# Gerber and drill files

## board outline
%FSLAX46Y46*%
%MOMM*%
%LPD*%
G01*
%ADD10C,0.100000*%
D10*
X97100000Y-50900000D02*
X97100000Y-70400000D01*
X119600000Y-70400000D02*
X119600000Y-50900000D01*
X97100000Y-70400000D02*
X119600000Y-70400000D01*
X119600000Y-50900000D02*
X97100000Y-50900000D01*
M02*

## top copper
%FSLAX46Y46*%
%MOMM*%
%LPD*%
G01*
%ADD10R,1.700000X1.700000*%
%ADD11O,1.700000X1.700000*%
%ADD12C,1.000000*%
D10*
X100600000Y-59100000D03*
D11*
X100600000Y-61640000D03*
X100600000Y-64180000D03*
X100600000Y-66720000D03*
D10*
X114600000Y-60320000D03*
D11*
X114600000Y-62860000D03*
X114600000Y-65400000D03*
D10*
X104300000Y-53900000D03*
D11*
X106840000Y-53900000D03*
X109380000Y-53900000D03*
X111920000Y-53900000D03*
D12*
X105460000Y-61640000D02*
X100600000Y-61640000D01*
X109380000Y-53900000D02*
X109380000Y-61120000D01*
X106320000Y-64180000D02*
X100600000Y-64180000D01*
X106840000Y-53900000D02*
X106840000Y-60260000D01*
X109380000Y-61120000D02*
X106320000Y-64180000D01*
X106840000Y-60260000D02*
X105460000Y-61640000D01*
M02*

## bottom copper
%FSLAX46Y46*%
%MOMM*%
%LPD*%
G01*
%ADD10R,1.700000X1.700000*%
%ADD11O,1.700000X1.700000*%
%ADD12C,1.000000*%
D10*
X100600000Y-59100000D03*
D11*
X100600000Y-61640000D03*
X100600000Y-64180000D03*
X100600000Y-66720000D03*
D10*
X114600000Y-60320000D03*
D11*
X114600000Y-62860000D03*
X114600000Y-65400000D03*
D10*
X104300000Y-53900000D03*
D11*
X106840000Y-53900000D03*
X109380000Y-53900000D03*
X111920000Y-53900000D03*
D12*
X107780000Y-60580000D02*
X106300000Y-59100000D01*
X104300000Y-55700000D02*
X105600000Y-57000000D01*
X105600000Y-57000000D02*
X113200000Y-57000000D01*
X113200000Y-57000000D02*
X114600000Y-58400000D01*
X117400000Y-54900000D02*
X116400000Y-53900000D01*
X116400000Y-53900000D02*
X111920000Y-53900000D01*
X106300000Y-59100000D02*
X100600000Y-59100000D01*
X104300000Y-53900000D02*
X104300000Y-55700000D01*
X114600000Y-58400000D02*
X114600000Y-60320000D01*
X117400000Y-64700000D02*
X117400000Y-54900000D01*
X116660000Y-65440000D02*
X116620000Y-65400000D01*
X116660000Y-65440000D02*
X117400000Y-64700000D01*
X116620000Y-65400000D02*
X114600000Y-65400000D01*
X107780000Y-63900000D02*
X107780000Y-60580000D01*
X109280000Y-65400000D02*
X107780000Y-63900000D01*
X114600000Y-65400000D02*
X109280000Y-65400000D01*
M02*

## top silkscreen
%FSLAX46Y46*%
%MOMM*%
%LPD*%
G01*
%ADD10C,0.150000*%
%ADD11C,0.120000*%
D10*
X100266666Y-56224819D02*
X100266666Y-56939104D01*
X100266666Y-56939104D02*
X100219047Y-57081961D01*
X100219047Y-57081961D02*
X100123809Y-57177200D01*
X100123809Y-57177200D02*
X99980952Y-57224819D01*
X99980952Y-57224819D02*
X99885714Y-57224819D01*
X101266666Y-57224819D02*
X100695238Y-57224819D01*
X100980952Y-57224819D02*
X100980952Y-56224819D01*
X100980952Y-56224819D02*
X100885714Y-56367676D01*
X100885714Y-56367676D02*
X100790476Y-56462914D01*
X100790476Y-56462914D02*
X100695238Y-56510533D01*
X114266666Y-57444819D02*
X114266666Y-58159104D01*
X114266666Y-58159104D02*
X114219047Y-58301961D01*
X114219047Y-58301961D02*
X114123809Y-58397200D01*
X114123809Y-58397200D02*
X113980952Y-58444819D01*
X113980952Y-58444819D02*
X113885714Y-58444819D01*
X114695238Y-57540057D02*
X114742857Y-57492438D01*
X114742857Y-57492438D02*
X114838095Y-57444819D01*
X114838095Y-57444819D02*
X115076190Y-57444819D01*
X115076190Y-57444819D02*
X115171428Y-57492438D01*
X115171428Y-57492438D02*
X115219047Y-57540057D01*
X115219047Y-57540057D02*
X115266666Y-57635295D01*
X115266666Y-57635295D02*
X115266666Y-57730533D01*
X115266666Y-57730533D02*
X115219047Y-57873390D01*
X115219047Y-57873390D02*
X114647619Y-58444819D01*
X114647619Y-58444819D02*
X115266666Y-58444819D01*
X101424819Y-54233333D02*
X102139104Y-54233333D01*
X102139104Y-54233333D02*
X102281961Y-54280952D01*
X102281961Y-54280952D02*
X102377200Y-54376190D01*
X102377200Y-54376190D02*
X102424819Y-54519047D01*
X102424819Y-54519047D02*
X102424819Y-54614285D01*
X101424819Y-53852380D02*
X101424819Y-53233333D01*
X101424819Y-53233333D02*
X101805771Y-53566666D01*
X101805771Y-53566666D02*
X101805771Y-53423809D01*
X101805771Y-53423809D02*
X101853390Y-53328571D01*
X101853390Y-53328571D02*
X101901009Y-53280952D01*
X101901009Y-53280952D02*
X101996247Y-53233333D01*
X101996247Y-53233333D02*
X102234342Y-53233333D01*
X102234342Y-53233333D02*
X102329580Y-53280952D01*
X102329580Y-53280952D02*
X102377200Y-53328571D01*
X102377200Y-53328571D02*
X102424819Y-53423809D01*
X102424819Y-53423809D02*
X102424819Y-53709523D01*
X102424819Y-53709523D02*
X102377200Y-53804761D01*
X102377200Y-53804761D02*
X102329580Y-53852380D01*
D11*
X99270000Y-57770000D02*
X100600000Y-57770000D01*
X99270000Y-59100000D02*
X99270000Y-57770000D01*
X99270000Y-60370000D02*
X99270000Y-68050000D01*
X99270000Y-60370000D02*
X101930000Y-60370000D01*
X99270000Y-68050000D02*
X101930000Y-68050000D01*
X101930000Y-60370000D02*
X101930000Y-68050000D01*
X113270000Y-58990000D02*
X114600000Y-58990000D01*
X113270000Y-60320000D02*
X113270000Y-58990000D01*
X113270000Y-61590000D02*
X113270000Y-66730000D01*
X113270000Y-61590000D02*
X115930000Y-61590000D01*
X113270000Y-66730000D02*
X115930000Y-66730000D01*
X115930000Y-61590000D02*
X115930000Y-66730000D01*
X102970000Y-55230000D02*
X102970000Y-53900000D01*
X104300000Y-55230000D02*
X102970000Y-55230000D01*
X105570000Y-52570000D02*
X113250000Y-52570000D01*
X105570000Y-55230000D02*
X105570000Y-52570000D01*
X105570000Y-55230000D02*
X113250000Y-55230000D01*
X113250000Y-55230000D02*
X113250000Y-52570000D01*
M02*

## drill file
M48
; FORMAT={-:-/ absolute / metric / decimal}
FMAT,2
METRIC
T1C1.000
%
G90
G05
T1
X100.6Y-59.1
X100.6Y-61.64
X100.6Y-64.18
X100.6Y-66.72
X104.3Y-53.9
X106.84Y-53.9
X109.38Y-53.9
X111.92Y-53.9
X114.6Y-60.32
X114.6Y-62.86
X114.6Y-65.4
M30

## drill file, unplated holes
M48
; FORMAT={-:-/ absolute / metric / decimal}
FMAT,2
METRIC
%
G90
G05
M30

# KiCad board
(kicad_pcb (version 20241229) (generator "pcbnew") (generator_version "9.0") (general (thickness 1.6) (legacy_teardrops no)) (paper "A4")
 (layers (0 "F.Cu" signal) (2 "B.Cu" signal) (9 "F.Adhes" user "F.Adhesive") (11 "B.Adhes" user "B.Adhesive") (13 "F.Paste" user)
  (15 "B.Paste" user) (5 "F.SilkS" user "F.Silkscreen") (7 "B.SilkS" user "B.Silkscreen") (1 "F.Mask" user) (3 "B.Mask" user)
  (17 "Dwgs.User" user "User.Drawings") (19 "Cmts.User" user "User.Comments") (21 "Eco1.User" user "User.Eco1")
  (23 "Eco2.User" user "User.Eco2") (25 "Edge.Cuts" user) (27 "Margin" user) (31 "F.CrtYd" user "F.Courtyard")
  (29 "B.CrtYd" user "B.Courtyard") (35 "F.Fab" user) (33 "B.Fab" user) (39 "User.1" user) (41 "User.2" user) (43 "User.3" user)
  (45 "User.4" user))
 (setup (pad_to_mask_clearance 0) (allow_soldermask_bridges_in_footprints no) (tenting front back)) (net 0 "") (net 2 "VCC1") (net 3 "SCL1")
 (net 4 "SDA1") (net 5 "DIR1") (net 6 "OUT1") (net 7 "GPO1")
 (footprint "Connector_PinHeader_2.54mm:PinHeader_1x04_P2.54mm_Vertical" (layer "F.Cu") (at 104.3 53.9 90)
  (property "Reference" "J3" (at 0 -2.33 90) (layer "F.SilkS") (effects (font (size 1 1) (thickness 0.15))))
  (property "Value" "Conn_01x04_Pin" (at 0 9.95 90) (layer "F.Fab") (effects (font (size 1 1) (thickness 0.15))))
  (fp_line (start -1.33 -1.33) (end 0 -1.33) (stroke (width 0.12) (type solid)) (layer "F.SilkS") (net 1))
  (fp_line (start -1.33 0) (end -1.33 -1.33) (stroke (width 0.12) (type solid)) (layer "F.SilkS") (net 1))
  (fp_line (start 1.33 1.27) (end 1.33 8.95) (stroke (width 0.12) (type solid)) (layer "F.SilkS") (net 1))
  (fp_line (start -1.33 1.27) (end 1.33 1.27) (stroke (width 0.12) (type solid)) (layer "F.SilkS") (net 1))
  (fp_line (start -1.33 1.27) (end -1.33 8.95) (stroke (width 0.12) (type solid)) (layer "F.SilkS") (net 1))
  (fp_line (start -1.33 8.95) (end 1.33 8.95) (stroke (width 0.12) (type solid)) (layer "F.SilkS") (net 1))
  (pad "1" thru_hole rect (at 0 0 90) (size 1.7 1.7) (drill 1) (layers "*.Cu" "*.Mask") (remove_unused_layers no) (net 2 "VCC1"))
  (pad "2" thru_hole oval (at 0 2.54 90) (size 1.7 1.7) (drill 1) (layers "*.Cu" "*.Mask") (remove_unused_layers no) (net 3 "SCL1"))
  (pad "3" thru_hole oval (at 0 5.08 90) (size 1.7 1.7) (drill 1) (layers "*.Cu" "*.Mask") (remove_unused_layers no) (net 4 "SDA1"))
  (pad "4" thru_hole oval (at 0 7.62 90) (size 1.7 1.7) (drill 1) (layers "*.Cu" "*.Mask") (remove_unused_layers no) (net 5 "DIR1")))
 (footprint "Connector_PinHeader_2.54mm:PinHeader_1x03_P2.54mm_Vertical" (layer "F.Cu") (at 114.6 60.32)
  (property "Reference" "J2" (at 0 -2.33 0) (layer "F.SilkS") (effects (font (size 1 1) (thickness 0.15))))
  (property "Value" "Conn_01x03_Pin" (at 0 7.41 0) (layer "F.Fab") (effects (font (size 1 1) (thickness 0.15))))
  (fp_line (start -1.33 -1.33) (end 0 -1.33) (stroke (width 0.12) (type solid)) (layer "F.SilkS") (net 1))
  (fp_line (start -1.33 0) (end -1.33 -1.33) (stroke (width 0.12) (type solid)) (layer "F.SilkS") (net 1))
  (fp_line (start -1.33 1.27) (end -1.33 6.41) (stroke (width 0.12) (type solid)) (layer "F.SilkS") (net 1))
  (fp_line (start -1.33 1.27) (end 1.33 1.27) (stroke (width 0.12) (type solid)) (layer "F.SilkS") (net 1))
  (fp_line (start -1.33 6.41) (end 1.33 6.41) (stroke (width 0.12) (type solid)) (layer "F.SilkS") (net 1))
  (fp_line (start 1.33 1.27) (end 1.33 6.41) (stroke (width 0.12) (type solid)) (layer "F.SilkS") (net 1))
  (pad "1" thru_hole rect (at 0 0) (size 1.7 1.7) (drill 1) (layers "*.Cu" "*.Mask") (remove_unused_layers no) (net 2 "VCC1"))
  (pad "2" thru_hole oval (at 0 2.54) (size 1.7 1.7) (drill 1) (layers "*.Cu" "*.Mask") (remove_unused_layers no) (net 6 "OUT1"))
  (pad "3" thru_hole oval (at 0 5.08) (size 1.7 1.7) (drill 1) (layers "*.Cu" "*.Mask") (remove_unused_layers no) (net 5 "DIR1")))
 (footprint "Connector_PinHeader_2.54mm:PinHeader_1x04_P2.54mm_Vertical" (layer "F.Cu") (at 100.6 59.1)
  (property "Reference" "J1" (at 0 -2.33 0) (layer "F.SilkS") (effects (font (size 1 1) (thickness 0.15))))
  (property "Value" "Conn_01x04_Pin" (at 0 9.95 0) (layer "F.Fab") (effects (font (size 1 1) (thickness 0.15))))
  (fp_line (start -1.33 -1.33) (end 0 -1.33) (stroke (width 0.12) (type solid)) (layer "F.SilkS") (net 1))
  (fp_line (start -1.33 0) (end -1.33 -1.33) (stroke (width 0.12) (type solid)) (layer "F.SilkS") (net 1))
  (fp_line (start -1.33 1.27) (end -1.33 8.95) (stroke (width 0.12) (type solid)) (layer "F.SilkS") (net 1))
  (fp_line (start -1.33 1.27) (end 1.33 1.27) (stroke (width 0.12) (type solid)) (layer "F.SilkS") (net 1))
  (fp_line (start -1.33 8.95) (end 1.33 8.95) (stroke (width 0.12) (type solid)) (layer "F.SilkS") (net 1))
  (fp_line (start 1.33 1.27) (end 1.33 8.95) (stroke (width 0.12) (type solid)) (layer "F.SilkS") (net 1))
  (pad "1" thru_hole rect (at 0 0) (size 1.7 1.7) (drill 1) (layers "*.Cu" "*.Mask") (remove_unused_layers no) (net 5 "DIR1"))
  (pad "2" thru_hole oval (at 0 2.54) (size 1.7 1.7) (drill 1) (layers "*.Cu" "*.Mask") (remove_unused_layers no) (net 3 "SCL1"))
  (pad "3" thru_hole oval (at 0 5.08) (size 1.7 1.7) (drill 1) (layers "*.Cu" "*.Mask") (remove_unused_layers no) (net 4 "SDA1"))
  (pad "4" thru_hole oval (at 0 7.62) (size 1.7 1.7) (drill 1) (layers "*.Cu" "*.Mask") (remove_unused_layers no) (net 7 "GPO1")))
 (gr_line (start 119.6 50.9) (end 97.1 50.9) (stroke (width 0.1) (type solid)) (layer "Edge.Cuts"))
 (gr_line (start 97.1 50.9) (end 97.1 70.4) (stroke (width 0.1) (type solid)) (layer "Edge.Cuts"))
 (gr_line (start 97.1 70.4) (end 119.6 70.4) (stroke (width 0.1) (type solid)) (layer "Edge.Cuts"))
 (gr_line (start 119.6 70.4) (end 119.6 50.9) (stroke (width 0.1) (type solid)) (layer "Edge.Cuts"))
 (segment (start 107.78 60.58) (end 106.3 59.1) (width 1) (layer "B.Cu") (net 5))
 (segment (start 117.4 54.9) (end 116.4 53.9) (width 1) (layer "B.Cu") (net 5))
 (segment (start 106.3 59.1) (end 100.6 59.1) (width 1) (layer "B.Cu") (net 5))
 (segment (start 116.4 53.9) (end 111.92 53.9) (width 1) (layer "B.Cu") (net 5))
 (segment (start 107.78 63.9) (end 107.78 60.58) (width 1) (layer "B.Cu") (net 5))
 (segment (start 109.28 65.4) (end 107.78 63.9) (width 1) (layer "B.Cu") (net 5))
 (segment (start 117.4 64.7) (end 117.4 54.9) (width 1) (layer "B.Cu") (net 5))
 (segment (start 116.66 65.44) (end 116.62 65.4) (width 1) (layer "B.Cu") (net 5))
 (segment (start 116.62 65.4) (end 114.6 65.4) (width 1) (layer "B.Cu") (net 5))
 (segment (start 116.66 65.44) (end 117.4 64.7) (width 1) (layer "B.Cu") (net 5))
 (segment (start 114.6 65.4) (end 109.28 65.4) (width 1) (layer "B.Cu") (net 5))
 (segment (start 106.84 60.26) (end 105.46 61.64) (width 1) (layer "F.Cu") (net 3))
 (segment (start 106.84 53.9) (end 106.84 60.26) (width 1) (layer "F.Cu") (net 3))
 (segment (start 105.46 61.64) (end 100.6 61.64) (width 1) (layer "F.Cu") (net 3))
 (segment (start 105.6 57) (end 113.2 57) (width 1) (layer "B.Cu") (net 2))
 (segment (start 114.6 58.4) (end 114.6 60.32) (width 1) (layer "B.Cu") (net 2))
 (segment (start 104.3 53.9) (end 104.3 55.7) (width 1) (layer "B.Cu") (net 2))
 (segment (start 113.2 57) (end 114.6 58.4) (width 1) (layer "B.Cu") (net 2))
 (segment (start 104.3 55.7) (end 105.6 57) (width 1) (layer "B.Cu") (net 2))
 (segment (start 109.38 61.12) (end 106.32 64.18) (width 1) (layer "F.Cu") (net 4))
 (segment (start 106.32 64.18) (end 100.6 64.18) (width 1) (layer "F.Cu") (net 4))
 (segment (start 109.38 53.9) (end 109.38 61.12) (width 1) (layer "F.Cu") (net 4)))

